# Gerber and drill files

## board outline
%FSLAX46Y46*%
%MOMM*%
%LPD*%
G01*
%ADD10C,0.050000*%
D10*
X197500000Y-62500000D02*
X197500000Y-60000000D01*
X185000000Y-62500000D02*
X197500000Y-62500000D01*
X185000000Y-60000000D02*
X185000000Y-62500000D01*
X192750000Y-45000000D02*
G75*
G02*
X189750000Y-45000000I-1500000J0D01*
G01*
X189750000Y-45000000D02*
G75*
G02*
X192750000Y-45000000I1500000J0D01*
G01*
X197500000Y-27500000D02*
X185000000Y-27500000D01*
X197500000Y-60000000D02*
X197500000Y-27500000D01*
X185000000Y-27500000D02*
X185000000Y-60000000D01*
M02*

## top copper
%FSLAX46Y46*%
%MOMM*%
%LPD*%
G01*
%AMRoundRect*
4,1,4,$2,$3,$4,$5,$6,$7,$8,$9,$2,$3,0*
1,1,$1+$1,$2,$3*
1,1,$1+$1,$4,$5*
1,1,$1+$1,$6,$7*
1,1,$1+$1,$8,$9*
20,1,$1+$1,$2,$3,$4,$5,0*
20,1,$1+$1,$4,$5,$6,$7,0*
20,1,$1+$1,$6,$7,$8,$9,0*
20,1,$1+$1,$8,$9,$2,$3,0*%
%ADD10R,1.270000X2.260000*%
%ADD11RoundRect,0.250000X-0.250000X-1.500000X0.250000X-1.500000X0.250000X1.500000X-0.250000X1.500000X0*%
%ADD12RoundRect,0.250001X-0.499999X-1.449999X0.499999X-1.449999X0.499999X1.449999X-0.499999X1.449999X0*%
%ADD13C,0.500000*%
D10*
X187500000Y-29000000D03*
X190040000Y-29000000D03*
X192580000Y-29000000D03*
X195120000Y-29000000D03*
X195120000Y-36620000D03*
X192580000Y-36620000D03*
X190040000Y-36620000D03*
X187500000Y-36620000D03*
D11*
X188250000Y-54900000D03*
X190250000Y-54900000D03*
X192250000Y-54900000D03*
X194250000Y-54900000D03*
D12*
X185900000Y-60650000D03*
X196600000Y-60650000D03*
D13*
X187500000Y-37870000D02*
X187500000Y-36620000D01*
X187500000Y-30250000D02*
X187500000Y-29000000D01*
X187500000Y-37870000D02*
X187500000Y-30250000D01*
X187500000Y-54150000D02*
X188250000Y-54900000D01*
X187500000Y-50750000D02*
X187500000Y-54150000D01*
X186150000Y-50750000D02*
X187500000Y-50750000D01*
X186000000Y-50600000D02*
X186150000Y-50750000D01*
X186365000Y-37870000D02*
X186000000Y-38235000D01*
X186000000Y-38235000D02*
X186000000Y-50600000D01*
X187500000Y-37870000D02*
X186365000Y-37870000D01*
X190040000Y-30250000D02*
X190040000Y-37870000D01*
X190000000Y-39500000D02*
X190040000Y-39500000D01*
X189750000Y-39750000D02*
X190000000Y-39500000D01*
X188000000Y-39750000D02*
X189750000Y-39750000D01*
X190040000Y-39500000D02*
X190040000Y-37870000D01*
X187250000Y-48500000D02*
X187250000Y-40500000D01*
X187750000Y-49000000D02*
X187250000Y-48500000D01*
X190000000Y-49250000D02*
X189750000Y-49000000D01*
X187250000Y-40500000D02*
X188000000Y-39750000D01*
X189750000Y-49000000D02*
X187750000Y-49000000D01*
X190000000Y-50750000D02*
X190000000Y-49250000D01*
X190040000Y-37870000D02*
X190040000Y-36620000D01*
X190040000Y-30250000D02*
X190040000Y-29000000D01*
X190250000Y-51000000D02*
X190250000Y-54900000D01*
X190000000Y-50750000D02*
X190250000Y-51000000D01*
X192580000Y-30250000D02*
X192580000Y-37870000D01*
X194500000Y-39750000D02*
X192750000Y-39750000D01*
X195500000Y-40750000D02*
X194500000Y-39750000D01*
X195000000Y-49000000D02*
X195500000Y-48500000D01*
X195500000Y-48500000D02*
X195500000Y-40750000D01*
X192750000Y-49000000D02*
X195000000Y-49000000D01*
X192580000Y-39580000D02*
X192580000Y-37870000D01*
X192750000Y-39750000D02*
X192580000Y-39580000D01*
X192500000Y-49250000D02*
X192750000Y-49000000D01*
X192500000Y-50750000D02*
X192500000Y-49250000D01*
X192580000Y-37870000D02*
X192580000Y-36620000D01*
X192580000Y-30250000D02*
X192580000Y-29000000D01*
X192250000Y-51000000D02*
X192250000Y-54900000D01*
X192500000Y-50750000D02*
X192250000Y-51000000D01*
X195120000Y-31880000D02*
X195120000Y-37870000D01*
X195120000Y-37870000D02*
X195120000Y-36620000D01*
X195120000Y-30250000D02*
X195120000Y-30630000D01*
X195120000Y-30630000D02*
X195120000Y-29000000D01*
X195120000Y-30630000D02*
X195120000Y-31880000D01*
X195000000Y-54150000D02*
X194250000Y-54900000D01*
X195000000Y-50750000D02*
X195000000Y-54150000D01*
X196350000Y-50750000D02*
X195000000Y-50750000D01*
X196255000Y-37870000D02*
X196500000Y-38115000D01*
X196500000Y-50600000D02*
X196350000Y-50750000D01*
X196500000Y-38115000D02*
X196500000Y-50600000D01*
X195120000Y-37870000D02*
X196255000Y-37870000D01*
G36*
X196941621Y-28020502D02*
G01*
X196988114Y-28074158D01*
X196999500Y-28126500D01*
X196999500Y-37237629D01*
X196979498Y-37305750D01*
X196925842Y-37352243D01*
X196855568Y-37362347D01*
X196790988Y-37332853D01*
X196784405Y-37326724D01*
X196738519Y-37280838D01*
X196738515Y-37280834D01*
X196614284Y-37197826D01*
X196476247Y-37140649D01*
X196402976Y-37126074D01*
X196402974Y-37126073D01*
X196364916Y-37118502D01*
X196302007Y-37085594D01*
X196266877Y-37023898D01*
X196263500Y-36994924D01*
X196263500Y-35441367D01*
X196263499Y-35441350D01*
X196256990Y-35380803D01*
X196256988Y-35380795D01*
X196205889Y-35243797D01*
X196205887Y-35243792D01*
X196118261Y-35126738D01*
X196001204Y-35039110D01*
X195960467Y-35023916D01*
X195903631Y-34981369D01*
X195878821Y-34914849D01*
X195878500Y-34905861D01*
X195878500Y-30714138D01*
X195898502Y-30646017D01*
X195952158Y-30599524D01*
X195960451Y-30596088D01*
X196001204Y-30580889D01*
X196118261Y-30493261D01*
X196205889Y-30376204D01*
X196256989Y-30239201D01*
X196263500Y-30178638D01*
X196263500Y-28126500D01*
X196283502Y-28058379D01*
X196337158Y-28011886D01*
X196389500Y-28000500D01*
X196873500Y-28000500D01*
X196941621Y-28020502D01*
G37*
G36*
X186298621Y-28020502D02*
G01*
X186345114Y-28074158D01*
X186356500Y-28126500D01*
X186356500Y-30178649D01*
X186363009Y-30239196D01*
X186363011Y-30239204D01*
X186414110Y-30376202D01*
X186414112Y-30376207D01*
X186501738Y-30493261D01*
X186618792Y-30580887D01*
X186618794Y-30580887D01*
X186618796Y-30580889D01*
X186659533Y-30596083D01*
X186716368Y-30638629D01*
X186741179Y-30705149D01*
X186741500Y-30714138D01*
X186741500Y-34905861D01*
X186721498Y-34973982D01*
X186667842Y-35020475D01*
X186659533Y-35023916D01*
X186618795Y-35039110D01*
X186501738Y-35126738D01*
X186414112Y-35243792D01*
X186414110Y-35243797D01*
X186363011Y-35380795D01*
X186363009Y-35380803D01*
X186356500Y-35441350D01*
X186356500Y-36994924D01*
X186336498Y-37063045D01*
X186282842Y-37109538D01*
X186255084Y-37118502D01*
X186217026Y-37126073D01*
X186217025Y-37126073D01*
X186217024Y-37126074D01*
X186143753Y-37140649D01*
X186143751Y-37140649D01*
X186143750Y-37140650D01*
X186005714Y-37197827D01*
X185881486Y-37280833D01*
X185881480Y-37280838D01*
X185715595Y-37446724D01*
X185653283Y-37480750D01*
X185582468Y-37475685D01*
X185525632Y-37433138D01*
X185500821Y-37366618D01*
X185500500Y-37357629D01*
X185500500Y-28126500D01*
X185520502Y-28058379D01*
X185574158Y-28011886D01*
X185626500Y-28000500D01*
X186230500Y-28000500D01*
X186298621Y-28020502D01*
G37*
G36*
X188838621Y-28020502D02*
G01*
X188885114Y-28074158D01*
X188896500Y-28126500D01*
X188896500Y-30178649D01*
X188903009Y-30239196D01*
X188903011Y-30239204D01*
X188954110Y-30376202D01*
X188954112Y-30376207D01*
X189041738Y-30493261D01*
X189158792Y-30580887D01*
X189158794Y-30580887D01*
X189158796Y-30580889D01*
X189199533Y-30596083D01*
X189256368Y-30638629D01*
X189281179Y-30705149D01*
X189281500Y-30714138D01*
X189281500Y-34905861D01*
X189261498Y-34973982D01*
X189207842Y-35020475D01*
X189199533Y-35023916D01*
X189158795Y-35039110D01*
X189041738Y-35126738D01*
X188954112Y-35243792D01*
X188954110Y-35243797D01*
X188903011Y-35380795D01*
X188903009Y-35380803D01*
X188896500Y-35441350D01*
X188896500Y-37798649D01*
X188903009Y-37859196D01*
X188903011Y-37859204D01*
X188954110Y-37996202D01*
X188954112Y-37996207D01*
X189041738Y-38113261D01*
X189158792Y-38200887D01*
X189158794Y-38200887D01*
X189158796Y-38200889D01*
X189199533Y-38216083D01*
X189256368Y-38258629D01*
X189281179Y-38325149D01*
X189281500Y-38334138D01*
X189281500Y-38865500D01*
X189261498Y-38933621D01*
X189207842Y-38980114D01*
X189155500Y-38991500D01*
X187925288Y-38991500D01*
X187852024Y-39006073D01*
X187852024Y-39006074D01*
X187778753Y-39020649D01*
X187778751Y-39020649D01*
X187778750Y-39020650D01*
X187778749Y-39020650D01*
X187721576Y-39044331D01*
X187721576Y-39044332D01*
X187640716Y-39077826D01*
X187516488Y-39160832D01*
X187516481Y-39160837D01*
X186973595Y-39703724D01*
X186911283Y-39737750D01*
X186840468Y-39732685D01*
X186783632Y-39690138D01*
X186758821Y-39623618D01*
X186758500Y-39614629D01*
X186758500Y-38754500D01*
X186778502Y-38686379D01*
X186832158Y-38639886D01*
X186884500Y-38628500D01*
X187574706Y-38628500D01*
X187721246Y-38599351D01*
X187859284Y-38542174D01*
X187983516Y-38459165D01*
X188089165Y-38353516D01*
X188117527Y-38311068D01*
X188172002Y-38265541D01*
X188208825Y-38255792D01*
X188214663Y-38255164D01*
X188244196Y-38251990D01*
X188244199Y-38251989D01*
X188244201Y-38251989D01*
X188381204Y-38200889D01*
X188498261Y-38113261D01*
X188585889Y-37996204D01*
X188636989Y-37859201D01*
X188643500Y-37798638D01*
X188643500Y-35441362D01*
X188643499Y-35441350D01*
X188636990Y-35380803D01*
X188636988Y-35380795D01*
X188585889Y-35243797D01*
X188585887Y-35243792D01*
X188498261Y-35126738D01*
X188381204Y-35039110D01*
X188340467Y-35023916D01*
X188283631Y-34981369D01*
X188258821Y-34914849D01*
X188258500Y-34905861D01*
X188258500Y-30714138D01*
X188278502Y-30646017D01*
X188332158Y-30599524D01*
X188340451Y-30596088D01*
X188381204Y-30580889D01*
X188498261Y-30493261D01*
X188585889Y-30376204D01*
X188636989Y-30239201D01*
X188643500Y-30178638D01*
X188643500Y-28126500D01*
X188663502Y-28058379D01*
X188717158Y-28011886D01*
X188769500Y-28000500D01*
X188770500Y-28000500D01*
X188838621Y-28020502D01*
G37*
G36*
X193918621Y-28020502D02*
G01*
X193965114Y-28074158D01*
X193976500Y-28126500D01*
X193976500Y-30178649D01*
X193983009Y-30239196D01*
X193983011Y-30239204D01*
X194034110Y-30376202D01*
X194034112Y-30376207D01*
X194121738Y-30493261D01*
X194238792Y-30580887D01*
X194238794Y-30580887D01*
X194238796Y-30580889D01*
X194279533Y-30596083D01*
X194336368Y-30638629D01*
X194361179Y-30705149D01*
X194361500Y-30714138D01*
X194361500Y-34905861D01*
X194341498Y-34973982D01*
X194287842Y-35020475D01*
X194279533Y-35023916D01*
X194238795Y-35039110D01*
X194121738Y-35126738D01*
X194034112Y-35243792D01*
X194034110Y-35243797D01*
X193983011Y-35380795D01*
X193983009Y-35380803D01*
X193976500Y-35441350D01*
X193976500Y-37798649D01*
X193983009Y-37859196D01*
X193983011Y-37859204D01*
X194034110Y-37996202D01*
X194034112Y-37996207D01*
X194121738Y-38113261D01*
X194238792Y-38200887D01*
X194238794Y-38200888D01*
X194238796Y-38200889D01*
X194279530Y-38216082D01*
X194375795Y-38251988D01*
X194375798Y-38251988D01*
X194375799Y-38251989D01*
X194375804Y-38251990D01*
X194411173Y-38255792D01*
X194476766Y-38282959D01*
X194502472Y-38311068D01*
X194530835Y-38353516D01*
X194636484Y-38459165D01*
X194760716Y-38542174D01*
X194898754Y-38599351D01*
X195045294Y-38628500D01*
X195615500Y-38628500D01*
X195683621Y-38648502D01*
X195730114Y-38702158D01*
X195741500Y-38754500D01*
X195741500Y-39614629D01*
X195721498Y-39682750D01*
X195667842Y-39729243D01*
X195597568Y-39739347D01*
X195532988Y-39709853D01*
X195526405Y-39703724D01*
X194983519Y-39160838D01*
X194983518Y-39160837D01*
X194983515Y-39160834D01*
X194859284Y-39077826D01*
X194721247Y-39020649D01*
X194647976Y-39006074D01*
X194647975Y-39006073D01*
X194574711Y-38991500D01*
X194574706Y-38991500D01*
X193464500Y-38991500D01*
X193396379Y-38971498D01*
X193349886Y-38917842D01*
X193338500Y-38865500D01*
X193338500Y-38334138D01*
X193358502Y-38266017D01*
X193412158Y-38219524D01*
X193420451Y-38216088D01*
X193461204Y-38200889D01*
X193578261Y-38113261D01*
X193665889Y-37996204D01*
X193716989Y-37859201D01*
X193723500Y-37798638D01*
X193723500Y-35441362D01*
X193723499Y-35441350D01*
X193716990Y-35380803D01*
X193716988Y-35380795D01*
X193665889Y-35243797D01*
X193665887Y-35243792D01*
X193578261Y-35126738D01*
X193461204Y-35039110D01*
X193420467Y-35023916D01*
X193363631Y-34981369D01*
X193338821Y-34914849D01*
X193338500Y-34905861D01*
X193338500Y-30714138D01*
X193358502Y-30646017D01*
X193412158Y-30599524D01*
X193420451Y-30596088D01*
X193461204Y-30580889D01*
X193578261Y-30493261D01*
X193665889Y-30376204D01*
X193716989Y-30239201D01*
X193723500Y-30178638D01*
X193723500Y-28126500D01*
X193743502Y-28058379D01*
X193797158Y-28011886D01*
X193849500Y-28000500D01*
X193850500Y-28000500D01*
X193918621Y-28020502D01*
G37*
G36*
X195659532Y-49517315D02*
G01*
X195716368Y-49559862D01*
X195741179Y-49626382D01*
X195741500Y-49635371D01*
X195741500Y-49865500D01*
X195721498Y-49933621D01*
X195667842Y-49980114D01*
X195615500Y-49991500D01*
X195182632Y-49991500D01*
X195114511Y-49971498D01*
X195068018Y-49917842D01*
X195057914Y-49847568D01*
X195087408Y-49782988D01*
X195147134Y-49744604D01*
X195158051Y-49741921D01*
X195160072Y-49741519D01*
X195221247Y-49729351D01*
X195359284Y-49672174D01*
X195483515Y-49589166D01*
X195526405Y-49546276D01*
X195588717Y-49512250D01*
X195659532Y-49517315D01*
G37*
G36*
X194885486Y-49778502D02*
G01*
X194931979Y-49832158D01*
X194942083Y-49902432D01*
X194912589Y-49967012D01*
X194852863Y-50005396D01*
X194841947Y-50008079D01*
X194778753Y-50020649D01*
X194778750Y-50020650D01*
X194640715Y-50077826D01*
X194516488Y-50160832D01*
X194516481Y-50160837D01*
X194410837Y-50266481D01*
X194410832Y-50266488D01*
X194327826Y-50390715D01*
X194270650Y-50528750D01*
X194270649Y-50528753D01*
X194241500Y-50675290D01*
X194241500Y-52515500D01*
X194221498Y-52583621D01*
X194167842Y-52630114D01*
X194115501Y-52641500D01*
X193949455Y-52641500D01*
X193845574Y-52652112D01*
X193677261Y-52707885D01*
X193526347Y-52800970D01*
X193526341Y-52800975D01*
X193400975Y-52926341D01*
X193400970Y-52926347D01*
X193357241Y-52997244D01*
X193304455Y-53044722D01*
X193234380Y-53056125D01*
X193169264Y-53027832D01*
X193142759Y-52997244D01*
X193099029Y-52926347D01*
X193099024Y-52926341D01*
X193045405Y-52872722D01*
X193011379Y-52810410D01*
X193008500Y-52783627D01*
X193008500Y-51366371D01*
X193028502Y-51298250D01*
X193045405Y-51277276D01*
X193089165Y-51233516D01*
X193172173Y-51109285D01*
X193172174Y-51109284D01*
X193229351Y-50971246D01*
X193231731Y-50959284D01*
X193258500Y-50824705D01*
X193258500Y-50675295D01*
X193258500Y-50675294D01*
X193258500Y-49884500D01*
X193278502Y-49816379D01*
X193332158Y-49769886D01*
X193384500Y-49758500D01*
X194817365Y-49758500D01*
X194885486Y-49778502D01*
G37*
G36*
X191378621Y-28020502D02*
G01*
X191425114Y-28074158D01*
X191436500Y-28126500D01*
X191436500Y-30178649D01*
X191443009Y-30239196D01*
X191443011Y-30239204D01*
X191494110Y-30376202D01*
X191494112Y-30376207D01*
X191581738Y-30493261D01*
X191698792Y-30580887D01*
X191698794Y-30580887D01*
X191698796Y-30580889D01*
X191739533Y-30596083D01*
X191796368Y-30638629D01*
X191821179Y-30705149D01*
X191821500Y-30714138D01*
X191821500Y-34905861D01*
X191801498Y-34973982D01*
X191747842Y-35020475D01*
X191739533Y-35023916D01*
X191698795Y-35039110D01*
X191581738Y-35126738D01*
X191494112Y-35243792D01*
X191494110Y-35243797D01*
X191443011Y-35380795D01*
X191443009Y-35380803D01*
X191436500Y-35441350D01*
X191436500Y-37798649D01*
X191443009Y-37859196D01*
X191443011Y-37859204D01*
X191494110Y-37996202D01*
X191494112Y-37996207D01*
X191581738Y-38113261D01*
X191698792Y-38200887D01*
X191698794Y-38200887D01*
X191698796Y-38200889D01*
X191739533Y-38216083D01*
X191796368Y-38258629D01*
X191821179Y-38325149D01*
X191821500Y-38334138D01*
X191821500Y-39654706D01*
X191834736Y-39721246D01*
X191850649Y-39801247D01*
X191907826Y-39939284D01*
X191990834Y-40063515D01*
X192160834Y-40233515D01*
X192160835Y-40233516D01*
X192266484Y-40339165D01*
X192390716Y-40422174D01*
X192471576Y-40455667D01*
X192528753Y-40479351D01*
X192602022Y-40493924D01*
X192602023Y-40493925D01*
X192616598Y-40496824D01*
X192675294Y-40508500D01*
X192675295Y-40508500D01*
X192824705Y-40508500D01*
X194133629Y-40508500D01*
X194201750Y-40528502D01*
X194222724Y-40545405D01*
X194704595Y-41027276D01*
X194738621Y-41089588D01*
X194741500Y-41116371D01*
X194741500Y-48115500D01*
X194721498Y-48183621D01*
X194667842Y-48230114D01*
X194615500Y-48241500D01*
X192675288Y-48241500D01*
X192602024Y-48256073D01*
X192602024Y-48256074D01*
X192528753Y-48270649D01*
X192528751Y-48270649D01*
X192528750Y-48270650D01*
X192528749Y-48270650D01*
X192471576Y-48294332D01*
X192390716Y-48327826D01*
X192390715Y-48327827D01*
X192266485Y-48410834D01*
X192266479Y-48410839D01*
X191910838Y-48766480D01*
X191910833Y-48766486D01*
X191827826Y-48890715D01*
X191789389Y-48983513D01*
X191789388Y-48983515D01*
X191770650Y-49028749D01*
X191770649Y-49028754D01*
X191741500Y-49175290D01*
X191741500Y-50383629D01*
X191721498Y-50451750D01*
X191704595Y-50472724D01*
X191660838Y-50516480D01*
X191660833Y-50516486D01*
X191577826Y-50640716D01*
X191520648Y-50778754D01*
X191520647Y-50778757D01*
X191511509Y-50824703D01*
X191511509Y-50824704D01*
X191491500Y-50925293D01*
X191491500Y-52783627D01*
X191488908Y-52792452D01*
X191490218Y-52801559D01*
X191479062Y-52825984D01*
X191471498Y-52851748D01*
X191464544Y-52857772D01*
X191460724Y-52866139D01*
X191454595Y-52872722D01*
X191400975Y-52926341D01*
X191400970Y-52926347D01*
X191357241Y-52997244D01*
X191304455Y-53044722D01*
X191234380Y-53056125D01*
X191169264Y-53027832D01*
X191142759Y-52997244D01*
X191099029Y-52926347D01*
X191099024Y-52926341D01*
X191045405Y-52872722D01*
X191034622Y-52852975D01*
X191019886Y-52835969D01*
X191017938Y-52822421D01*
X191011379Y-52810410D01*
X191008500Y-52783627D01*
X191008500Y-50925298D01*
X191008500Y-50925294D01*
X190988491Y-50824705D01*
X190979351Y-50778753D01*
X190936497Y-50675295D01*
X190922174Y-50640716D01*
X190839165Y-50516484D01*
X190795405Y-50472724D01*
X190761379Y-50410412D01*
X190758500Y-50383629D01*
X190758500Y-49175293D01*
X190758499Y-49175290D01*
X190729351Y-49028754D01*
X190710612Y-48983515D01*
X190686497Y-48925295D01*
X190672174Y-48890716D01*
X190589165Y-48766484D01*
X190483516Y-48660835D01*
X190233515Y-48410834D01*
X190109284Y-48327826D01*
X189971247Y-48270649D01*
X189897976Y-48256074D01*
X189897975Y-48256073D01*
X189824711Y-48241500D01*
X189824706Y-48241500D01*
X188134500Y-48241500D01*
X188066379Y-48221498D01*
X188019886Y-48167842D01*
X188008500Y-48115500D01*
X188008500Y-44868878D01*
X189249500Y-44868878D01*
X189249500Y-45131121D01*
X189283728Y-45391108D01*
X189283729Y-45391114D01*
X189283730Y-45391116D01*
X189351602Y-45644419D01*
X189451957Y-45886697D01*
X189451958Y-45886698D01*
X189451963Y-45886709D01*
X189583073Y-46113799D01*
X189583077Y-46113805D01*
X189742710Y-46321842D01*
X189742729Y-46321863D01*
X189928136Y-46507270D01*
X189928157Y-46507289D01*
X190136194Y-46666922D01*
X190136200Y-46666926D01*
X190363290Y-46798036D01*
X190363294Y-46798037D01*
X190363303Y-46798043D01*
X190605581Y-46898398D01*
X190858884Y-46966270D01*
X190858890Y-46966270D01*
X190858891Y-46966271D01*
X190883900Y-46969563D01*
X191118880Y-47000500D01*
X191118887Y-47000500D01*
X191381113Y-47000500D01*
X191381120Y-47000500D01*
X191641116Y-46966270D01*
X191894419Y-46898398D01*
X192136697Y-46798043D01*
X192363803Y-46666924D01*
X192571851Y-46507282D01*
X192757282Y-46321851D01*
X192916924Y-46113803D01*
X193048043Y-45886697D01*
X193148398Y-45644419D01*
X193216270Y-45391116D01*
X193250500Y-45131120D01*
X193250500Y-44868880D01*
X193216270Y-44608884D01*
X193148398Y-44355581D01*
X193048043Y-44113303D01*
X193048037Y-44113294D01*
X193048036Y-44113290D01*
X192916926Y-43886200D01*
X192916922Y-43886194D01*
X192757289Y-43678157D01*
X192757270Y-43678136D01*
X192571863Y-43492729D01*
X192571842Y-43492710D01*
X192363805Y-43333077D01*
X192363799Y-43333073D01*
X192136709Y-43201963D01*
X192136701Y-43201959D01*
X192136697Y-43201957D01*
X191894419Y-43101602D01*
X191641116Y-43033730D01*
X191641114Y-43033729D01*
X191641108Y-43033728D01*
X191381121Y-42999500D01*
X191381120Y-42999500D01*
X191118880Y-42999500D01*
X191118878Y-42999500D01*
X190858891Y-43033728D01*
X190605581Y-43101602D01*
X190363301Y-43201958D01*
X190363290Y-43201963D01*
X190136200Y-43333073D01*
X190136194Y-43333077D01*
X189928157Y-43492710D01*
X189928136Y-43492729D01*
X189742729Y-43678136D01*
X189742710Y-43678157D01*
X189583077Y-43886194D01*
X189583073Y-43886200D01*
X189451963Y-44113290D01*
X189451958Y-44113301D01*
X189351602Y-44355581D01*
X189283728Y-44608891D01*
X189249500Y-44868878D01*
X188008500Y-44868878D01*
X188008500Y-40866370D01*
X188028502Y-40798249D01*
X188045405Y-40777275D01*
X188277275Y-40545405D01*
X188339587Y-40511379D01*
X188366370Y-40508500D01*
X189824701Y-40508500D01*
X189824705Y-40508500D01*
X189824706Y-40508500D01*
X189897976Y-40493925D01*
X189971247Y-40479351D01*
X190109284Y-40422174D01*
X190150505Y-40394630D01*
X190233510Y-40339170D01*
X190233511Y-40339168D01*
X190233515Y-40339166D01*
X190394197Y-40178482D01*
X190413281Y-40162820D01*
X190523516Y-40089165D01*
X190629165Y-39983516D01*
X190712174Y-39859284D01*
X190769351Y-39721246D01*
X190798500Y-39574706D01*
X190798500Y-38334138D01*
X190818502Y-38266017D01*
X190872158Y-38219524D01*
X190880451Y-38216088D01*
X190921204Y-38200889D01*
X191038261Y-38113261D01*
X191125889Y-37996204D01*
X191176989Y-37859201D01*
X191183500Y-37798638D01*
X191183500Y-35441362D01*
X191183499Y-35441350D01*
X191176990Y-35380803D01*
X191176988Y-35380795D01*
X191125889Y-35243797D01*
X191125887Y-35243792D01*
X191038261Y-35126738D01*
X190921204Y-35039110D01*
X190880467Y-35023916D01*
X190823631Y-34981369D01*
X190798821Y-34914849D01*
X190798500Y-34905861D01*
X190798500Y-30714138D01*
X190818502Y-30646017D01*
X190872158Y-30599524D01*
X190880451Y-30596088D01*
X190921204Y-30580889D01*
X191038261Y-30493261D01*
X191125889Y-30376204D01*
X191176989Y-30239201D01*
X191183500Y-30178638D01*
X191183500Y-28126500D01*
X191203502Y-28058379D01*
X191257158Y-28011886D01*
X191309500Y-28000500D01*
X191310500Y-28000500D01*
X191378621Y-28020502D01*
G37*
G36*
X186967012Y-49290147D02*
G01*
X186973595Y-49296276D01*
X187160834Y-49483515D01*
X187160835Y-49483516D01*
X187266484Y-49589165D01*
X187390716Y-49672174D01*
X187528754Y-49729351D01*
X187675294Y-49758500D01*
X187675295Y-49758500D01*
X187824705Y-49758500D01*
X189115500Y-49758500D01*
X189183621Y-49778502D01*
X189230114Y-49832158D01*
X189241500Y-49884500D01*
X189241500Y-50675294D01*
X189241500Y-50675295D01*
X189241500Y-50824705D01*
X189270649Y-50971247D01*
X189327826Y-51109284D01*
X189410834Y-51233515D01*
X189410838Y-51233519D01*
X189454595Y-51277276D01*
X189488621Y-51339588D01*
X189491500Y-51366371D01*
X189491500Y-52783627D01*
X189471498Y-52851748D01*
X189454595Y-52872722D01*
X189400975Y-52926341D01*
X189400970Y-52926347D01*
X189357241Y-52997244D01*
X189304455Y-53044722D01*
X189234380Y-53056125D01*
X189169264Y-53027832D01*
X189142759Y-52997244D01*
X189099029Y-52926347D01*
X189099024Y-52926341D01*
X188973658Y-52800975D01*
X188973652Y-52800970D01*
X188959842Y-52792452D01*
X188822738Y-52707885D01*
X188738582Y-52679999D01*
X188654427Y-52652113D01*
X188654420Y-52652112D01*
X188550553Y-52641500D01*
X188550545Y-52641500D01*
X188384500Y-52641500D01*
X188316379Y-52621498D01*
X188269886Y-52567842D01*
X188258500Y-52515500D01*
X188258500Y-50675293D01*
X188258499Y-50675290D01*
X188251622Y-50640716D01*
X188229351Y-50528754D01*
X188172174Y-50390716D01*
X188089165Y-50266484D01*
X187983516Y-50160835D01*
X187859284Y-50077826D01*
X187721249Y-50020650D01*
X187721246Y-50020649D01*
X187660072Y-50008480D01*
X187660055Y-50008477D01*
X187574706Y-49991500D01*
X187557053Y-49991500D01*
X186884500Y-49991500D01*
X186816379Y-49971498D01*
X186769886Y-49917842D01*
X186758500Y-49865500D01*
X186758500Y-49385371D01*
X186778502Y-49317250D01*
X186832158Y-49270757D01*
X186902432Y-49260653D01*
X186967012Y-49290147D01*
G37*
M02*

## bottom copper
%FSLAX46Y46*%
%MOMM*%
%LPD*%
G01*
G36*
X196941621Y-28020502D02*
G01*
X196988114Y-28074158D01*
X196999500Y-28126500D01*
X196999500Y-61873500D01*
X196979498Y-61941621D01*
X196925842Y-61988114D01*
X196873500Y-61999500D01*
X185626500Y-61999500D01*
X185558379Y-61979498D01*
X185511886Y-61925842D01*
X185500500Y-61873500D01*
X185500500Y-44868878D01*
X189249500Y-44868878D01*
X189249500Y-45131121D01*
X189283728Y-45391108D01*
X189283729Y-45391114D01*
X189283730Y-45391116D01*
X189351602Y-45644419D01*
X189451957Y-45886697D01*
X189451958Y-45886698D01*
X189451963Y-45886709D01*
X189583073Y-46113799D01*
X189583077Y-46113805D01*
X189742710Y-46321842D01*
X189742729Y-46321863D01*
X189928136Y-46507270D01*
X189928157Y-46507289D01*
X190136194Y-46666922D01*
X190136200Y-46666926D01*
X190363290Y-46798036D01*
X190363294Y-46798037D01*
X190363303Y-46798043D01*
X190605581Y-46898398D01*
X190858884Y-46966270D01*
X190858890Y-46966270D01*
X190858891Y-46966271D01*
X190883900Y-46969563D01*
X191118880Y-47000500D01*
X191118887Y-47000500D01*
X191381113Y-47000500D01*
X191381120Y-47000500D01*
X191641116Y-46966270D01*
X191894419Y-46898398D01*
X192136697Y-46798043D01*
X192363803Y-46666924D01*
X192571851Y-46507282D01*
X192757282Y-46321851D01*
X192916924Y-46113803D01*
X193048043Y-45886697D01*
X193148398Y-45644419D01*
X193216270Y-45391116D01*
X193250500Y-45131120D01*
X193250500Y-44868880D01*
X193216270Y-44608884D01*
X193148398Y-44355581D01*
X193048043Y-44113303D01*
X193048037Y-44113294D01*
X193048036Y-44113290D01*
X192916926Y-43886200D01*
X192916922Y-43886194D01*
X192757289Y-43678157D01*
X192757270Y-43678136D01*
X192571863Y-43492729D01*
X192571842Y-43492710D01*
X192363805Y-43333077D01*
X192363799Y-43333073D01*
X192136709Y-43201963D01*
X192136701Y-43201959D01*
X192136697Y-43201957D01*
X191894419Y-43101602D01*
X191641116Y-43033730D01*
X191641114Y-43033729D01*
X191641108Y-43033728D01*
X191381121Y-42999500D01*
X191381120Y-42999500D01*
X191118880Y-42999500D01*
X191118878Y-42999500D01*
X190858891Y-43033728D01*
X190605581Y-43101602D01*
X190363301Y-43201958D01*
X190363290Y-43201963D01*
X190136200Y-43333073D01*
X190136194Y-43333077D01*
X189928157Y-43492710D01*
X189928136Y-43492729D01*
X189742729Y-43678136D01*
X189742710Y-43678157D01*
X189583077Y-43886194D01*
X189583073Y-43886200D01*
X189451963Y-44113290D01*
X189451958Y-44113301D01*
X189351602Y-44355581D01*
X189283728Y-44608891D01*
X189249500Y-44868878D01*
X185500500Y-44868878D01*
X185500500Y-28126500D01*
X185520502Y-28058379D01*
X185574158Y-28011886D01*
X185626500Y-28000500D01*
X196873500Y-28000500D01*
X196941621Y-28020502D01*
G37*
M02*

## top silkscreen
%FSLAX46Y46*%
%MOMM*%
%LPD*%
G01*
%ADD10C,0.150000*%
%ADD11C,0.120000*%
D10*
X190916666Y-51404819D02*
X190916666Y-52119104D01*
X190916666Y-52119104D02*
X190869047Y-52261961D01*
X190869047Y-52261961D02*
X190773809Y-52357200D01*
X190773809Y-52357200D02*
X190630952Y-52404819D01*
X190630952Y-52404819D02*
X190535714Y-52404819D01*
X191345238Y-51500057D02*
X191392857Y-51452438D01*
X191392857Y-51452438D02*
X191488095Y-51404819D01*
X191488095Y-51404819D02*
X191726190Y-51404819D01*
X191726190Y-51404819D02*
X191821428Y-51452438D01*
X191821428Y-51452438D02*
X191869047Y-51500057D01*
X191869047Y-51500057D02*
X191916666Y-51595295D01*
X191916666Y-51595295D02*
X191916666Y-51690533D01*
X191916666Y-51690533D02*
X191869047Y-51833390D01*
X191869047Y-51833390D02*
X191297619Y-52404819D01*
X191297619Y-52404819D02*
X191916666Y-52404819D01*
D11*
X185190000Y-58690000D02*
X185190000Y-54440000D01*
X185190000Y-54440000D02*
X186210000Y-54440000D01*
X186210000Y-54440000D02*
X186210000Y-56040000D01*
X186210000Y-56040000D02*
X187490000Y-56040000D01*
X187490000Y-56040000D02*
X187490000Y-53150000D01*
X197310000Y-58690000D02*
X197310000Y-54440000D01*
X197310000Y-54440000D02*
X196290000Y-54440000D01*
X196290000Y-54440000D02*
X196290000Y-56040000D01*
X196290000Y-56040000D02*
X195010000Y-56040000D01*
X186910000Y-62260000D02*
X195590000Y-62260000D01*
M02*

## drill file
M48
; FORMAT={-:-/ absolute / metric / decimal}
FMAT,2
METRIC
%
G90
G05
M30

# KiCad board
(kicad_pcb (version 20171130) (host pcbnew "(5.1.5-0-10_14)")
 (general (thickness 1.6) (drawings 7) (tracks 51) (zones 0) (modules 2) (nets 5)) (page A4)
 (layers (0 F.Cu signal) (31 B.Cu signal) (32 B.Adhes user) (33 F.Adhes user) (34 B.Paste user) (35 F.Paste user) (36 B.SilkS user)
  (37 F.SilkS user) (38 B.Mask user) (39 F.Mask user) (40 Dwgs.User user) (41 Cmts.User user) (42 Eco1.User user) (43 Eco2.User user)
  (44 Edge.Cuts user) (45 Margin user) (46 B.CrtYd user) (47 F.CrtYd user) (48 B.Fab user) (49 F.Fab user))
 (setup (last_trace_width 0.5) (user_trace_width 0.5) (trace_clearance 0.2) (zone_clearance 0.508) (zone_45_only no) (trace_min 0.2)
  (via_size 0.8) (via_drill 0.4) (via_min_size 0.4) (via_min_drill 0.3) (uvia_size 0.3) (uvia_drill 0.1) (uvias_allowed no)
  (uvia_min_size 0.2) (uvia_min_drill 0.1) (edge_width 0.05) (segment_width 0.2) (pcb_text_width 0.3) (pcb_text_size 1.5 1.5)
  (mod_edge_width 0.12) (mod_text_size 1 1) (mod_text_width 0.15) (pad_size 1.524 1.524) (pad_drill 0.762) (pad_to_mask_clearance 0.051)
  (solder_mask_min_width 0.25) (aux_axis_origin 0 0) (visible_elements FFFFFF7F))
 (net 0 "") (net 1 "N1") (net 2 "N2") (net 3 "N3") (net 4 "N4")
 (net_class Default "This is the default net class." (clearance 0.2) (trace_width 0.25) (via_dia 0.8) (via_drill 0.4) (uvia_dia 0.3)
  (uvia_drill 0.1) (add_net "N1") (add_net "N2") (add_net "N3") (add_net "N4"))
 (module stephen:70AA (layer F.Cu) (at 187.5 29)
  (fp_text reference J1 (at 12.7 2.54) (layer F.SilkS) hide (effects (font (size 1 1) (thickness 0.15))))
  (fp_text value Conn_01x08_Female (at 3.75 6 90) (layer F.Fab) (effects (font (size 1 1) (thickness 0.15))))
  (pad 1 smd rect (at 0 0) (size 1.27 2.26) (layers F.Cu F.Paste F.Mask) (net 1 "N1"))
  (pad 2 smd rect (at 2.54 0) (size 1.27 2.26) (layers F.Cu F.Paste F.Mask) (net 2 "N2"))
  (pad 3 smd rect (at 5.08 0) (size 1.27 2.26) (layers F.Cu F.Paste F.Mask) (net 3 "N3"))
  (pad 4 smd rect (at 7.62 0) (size 1.27 2.26) (layers F.Cu F.Paste F.Mask) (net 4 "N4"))
  (pad 5 smd rect (at 7.62 7.62) (size 1.27 2.26) (layers F.Cu F.Paste F.Mask) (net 4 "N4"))
  (pad 6 smd rect (at 5.08 7.62) (size 1.27 2.26) (layers F.Cu F.Paste F.Mask) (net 3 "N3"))
  (pad 7 smd rect (at 2.54 7.62) (size 1.27 2.26) (layers F.Cu F.Paste F.Mask) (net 2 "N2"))
  (pad 8 smd rect (at 0 7.62) (size 1.27 2.26) (layers F.Cu F.Paste F.Mask) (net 1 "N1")))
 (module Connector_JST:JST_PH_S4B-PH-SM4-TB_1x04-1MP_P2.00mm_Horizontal (layer F.Cu) (at 191.25 57.75)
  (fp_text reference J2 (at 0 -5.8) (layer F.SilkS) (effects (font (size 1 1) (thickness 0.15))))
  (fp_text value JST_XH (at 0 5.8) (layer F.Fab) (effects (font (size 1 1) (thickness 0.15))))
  (fp_line (start -6.06 0.94) (end -6.06 -3.31) (layer F.SilkS) (width 0.12))
  (fp_line (start -6.06 -3.31) (end -5.04 -3.31) (layer F.SilkS) (width 0.12))
  (fp_line (start -5.04 -3.31) (end -5.04 -1.71) (layer F.SilkS) (width 0.12))
  (fp_line (start -5.04 -1.71) (end -3.76 -1.71) (layer F.SilkS) (width 0.12))
  (fp_line (start -3.76 -1.71) (end -3.76 -4.6) (layer F.SilkS) (width 0.12))
  (fp_line (start 6.06 0.94) (end 6.06 -3.31) (layer F.SilkS) (width 0.12))
  (fp_line (start 6.06 -3.31) (end 5.04 -3.31) (layer F.SilkS) (width 0.12))
  (fp_line (start 5.04 -3.31) (end 5.04 -1.71) (layer F.SilkS) (width 0.12))
  (fp_line (start 5.04 -1.71) (end 3.76 -1.71) (layer F.SilkS) (width 0.12))
  (fp_line (start -4.34 4.51) (end 4.34 4.51) (layer F.SilkS) (width 0.12))
  (pad 1 smd roundrect (at -3 -2.85) (size 1 3.5) (layers F.Cu F.Paste F.Mask) (roundrect_rratio 0.25) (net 1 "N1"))
  (pad 2 smd roundrect (at -1 -2.85) (size 1 3.5) (layers F.Cu F.Paste F.Mask) (roundrect_rratio 0.25) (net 2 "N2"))
  (pad 3 smd roundrect (at 1 -2.85) (size 1 3.5) (layers F.Cu F.Paste F.Mask) (roundrect_rratio 0.25) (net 3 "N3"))
  (pad 4 smd roundrect (at 3 -2.85) (size 1 3.5) (layers F.Cu F.Paste F.Mask) (roundrect_rratio 0.25) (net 4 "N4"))
  (pad MP smd roundrect (at -5.35 2.9) (size 1.5 3.4) (layers F.Cu F.Paste F.Mask) (roundrect_rratio 0.166667))
  (pad MP smd roundrect (at 5.35 2.9) (size 1.5 3.4) (layers F.Cu F.Paste F.Mask) (roundrect_rratio 0.166667)))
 (gr_line (start 197.5 62.5) (end 197.5 60) (layer Edge.Cuts) (width 0.05))
 (gr_line (start 185 62.5) (end 197.5 62.5) (layer Edge.Cuts) (width 0.05))
 (gr_line (start 185 60) (end 185 62.5) (layer Edge.Cuts) (width 0.05))
 (gr_circle (center 191.25 45) (end 192.75 45) (layer Edge.Cuts) (width 0.05))
 (gr_line (start 197.5 27.5) (end 185 27.5) (layer Edge.Cuts) (width 0.05))
 (gr_line (start 197.5 60) (end 197.5 27.5) (layer Edge.Cuts) (width 0.05))
 (gr_line (start 185 27.5) (end 185 60) (layer Edge.Cuts) (width 0.05))
 (segment (start 187.5 37.87) (end 187.5 36.62) (width 0.5) (layer F.Cu) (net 1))
 (segment (start 187.5 30.25) (end 187.5 29) (width 0.5) (layer F.Cu) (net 1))
 (segment (start 187.5 37.87) (end 187.5 30.25) (width 0.5) (layer F.Cu) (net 1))
 (segment (start 187.5 54.15) (end 188.25 54.9) (width 0.5) (layer F.Cu) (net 1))
 (segment (start 187.5 50.75) (end 187.5 54.15) (width 0.5) (layer F.Cu) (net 1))
 (segment (start 186.15 50.75) (end 187.5 50.75) (width 0.5) (layer F.Cu) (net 1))
 (segment (start 186 50.6) (end 186.15 50.75) (width 0.5) (layer F.Cu) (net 1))
 (segment (start 186.365 37.87) (end 186 38.235) (width 0.5) (layer F.Cu) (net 1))
 (segment (start 186 38.235) (end 186 50.6) (width 0.5) (layer F.Cu) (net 1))
 (segment (start 187.5 37.87) (end 186.365 37.87) (width 0.5) (layer F.Cu) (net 1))
 (segment (start 190.04 30.25) (end 190.04 37.87) (width 0.5) (layer F.Cu) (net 2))
 (segment (start 190 39.5) (end 190.04 39.5) (width 0.5) (layer F.Cu) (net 2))
 (segment (start 189.75 39.75) (end 190 39.5) (width 0.5) (layer F.Cu) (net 2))
 (segment (start 188 39.75) (end 189.75 39.75) (width 0.5) (layer F.Cu) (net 2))
 (segment (start 190.04 39.5) (end 190.04 37.87) (width 0.5) (layer F.Cu) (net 2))
 (segment (start 187.25 48.5) (end 187.25 40.5) (width 0.5) (layer F.Cu) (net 2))
 (segment (start 187.75 49) (end 187.25 48.5) (width 0.5) (layer F.Cu) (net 2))
 (segment (start 190 49.25) (end 189.75 49) (width 0.5) (layer F.Cu) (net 2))
 (segment (start 187.25 40.5) (end 188 39.75) (width 0.5) (layer F.Cu) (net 2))
 (segment (start 189.75 49) (end 187.75 49) (width 0.5) (layer F.Cu) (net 2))
 (segment (start 190 50.75) (end 190 49.25) (width 0.5) (layer F.Cu) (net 2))
 (segment (start 190.04 37.87) (end 190.04 36.62) (width 0.5) (layer F.Cu) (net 2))
 (segment (start 190.04 30.25) (end 190.04 29) (width 0.5) (layer F.Cu) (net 2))
 (segment (start 190.25 51) (end 190.25 54.9) (width 0.5) (layer F.Cu) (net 2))
 (segment (start 190 50.75) (end 190.25 51) (width 0.5) (layer F.Cu) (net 2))
 (segment (start 192.58 30.25) (end 192.58 37.87) (width 0.5) (layer F.Cu) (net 3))
 (segment (start 194.5 39.75) (end 192.75 39.75) (width 0.5) (layer F.Cu) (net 3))
 (segment (start 195.5 40.75) (end 194.5 39.75) (width 0.5) (layer F.Cu) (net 3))
 (segment (start 195 49) (end 195.5 48.5) (width 0.5) (layer F.Cu) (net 3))
 (segment (start 195.5 48.5) (end 195.5 40.75) (width 0.5) (layer F.Cu) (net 3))
 (segment (start 192.75 49) (end 195 49) (width 0.5) (layer F.Cu) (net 3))
 (segment (start 192.58 39.58) (end 192.58 37.87) (width 0.5) (layer F.Cu) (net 3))
 (segment (start 192.75 39.75) (end 192.58 39.58) (width 0.5) (layer F.Cu) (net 3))
 (segment (start 192.5 49.25) (end 192.75 49) (width 0.5) (layer F.Cu) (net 3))
 (segment (start 192.5 50.75) (end 192.5 49.25) (width 0.5) (layer F.Cu) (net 3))
 (segment (start 192.58 37.87) (end 192.58 36.62) (width 0.5) (layer F.Cu) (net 3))
 (segment (start 192.58 30.25) (end 192.58 29) (width 0.5) (layer F.Cu) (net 3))
 (segment (start 192.25 51) (end 192.25 54.9) (width 0.5) (layer F.Cu) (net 3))
 (segment (start 192.5 50.75) (end 192.25 51) (width 0.5) (layer F.Cu) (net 3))
 (segment (start 195.12 31.88) (end 195.12 37.87) (width 0.5) (layer F.Cu) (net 4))
 (segment (start 195.12 37.87) (end 195.12 36.62) (width 0.5) (layer F.Cu) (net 4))
 (segment (start 195.12 30.25) (end 195.12 30.63) (width 0.5) (layer F.Cu) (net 4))
 (segment (start 195.12 30.63) (end 195.12 29) (width 0.5) (layer F.Cu) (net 4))
 (segment (start 195.12 30.63) (end 195.12 31.88) (width 0.5) (layer F.Cu) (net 4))
 (segment (start 195 54.15) (end 194.25 54.9) (width 0.5) (layer F.Cu) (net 4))
 (segment (start 195 50.75) (end 195 54.15) (width 0.5) (layer F.Cu) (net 4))
 (segment (start 196.35 50.75) (end 195 50.75) (width 0.5) (layer F.Cu) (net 4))
 (segment (start 196.255 37.87) (end 196.5 38.115) (width 0.5) (layer F.Cu) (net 4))
 (segment (start 196.5 50.6) (end 196.35 50.75) (width 0.5) (layer F.Cu) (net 4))
 (segment (start 196.5 38.115) (end 196.5 50.6) (width 0.5) (layer F.Cu) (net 4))
 (segment (start 195.12 37.87) (end 196.255 37.87) (width 0.5) (layer F.Cu) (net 4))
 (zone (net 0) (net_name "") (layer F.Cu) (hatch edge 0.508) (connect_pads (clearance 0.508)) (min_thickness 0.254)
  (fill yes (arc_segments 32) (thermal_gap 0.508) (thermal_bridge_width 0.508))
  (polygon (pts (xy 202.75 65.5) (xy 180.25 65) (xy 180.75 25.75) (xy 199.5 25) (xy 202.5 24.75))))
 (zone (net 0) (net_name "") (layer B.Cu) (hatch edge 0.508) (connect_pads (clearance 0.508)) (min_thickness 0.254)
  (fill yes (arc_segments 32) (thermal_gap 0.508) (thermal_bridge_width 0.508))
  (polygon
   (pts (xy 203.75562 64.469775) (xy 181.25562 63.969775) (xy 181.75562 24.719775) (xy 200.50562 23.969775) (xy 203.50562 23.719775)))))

